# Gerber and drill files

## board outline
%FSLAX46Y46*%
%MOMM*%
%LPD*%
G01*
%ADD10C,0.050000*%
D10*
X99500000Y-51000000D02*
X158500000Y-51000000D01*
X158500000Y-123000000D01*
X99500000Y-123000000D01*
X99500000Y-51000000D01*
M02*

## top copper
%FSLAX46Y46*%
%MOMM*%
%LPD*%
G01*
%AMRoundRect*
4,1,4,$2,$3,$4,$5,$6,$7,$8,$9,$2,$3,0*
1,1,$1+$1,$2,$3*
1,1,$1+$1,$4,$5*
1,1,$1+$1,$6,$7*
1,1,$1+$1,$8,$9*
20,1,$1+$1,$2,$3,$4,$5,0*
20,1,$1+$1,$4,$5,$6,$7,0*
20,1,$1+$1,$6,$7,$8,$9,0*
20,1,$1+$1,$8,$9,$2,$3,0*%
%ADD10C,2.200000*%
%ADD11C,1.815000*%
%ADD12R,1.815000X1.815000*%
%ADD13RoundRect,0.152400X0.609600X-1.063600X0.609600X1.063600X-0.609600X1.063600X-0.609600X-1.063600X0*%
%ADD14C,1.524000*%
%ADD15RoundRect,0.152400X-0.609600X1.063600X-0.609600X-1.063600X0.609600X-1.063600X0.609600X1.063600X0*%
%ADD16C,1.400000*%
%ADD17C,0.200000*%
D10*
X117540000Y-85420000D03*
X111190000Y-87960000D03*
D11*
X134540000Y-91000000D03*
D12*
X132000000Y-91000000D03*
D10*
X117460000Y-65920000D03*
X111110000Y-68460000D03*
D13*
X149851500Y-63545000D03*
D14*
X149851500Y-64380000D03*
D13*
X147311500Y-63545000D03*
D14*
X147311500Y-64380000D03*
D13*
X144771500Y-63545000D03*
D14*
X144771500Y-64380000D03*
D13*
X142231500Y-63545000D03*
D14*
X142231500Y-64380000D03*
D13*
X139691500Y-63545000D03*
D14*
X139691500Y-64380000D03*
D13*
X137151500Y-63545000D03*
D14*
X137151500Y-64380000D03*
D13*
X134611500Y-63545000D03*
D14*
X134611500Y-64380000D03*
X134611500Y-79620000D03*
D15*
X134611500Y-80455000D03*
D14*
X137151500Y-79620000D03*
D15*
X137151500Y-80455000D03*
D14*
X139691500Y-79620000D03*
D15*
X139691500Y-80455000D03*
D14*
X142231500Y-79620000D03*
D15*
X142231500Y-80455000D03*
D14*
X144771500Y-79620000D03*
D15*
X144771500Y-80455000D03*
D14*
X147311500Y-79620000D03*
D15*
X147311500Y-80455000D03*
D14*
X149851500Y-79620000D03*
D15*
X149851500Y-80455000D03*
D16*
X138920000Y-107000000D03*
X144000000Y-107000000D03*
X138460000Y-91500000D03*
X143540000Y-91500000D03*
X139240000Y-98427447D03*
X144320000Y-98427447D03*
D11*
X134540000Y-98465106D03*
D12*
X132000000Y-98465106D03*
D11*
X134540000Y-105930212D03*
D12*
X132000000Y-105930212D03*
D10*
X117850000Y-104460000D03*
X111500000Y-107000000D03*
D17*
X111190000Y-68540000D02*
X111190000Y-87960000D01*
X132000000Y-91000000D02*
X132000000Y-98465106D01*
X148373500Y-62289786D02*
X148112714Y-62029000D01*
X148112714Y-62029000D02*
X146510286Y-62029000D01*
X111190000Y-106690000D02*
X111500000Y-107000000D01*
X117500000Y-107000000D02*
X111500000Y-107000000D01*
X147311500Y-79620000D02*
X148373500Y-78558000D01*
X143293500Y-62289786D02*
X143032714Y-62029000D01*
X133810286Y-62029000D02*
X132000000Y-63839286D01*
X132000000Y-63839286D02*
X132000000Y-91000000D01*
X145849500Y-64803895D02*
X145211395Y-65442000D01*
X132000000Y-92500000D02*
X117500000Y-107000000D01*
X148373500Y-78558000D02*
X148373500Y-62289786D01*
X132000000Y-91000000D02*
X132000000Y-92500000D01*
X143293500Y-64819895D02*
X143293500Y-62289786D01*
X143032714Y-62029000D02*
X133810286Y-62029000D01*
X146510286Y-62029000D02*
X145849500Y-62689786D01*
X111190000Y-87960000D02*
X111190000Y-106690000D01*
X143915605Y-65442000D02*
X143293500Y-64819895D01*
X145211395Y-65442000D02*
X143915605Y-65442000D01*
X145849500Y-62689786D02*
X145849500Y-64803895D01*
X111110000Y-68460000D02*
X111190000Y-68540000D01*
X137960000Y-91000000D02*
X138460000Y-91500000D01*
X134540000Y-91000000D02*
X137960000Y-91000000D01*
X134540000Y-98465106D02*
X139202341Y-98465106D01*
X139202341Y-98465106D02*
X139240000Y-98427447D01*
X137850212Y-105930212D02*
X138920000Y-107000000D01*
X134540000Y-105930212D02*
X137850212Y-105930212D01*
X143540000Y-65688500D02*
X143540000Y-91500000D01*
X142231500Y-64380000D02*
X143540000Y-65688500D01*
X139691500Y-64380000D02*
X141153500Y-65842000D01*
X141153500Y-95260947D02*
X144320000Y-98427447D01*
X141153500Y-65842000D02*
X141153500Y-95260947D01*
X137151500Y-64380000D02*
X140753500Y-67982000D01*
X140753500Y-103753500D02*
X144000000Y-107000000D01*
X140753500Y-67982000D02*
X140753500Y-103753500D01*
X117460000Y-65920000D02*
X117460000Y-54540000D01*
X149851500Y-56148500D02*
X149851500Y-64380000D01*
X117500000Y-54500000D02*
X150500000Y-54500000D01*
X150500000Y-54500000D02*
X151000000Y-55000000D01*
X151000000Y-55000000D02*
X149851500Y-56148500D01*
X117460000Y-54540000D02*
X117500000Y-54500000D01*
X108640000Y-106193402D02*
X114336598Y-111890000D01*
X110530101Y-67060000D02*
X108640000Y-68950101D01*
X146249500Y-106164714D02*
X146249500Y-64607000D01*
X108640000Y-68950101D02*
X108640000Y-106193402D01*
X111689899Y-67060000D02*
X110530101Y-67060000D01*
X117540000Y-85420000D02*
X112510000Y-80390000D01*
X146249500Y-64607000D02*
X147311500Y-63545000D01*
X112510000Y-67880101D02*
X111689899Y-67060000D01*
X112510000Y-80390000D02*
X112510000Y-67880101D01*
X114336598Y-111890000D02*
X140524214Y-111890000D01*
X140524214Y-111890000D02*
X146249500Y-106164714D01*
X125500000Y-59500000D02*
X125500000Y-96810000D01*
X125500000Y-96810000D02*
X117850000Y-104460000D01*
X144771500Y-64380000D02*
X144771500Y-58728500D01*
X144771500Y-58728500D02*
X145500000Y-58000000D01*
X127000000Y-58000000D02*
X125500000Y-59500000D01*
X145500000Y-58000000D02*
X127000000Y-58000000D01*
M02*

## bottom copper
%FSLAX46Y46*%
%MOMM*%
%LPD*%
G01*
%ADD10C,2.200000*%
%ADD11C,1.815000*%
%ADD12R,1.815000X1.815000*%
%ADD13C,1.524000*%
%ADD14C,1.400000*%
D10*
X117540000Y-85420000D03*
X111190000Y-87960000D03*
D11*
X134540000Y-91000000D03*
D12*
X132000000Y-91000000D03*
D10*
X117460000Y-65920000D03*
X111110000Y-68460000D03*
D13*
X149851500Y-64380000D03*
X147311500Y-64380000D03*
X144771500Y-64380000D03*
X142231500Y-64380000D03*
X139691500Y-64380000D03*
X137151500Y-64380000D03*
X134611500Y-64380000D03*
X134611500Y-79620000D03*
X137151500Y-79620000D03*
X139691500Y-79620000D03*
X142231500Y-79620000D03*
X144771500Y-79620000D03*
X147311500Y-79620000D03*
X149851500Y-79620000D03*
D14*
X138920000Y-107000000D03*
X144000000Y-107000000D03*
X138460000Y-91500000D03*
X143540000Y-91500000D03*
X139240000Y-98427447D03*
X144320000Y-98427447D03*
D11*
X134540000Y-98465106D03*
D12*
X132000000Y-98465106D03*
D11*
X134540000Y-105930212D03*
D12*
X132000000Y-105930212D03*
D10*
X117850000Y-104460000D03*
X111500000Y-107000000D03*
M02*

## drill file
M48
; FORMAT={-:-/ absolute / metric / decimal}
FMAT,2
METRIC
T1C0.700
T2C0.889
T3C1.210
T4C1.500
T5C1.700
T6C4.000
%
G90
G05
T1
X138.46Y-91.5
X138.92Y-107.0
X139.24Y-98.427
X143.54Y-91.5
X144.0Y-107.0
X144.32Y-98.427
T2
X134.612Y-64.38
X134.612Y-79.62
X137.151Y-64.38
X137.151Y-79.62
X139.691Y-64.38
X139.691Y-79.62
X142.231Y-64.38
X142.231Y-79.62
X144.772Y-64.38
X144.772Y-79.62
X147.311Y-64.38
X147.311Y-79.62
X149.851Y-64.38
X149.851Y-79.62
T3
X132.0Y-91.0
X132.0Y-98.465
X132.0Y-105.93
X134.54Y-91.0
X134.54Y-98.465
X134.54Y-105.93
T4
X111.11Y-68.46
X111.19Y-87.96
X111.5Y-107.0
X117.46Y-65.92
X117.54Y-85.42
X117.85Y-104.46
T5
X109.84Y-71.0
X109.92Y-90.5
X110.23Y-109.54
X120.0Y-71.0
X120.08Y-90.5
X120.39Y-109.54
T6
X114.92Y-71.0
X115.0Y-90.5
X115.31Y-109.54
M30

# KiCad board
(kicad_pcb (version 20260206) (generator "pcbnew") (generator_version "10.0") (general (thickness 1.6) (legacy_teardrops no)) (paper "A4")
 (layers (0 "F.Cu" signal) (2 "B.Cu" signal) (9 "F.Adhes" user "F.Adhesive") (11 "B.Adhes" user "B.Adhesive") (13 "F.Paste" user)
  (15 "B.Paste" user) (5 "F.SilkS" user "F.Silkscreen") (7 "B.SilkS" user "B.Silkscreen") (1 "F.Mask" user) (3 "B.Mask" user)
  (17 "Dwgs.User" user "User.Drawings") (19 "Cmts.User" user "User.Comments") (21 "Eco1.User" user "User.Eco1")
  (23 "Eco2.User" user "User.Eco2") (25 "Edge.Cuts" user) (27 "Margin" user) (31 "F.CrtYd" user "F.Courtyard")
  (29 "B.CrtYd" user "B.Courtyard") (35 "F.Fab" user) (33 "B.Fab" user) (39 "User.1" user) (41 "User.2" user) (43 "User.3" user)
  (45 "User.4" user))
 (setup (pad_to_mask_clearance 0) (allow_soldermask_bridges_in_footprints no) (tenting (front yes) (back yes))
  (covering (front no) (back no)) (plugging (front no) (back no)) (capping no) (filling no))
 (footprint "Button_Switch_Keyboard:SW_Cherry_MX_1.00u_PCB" (layer "F.Cu") (at 117.54 85.42)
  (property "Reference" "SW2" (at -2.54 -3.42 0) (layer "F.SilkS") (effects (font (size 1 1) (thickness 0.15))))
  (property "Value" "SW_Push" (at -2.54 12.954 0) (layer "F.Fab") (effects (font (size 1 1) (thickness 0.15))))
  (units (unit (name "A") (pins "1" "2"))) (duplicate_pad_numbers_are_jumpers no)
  (pad "" np_thru_hole circle (at -7.62 5.08) (size 1.7 1.7) (drill 1.7) (layers "*.Cu" "*.Mask"))
  (pad "" np_thru_hole circle (at -2.54 5.08) (size 4 4) (drill 4) (layers "*.Cu" "*.Mask"))
  (pad "" np_thru_hole circle (at 2.54 5.08) (size 1.7 1.7) (drill 1.7) (layers "*.Cu" "*.Mask"))
  (pad "1" thru_hole circle (at 0 0) (size 2.2 2.2) (drill 1.5) (layers "*.Cu" "*.Mask") (remove_unused_layers no) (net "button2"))
  (pad "2" thru_hole circle (at -6.35 2.54) (size 2.2 2.2) (drill 1.5) (layers "*.Cu" "*.Mask") (remove_unused_layers no) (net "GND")))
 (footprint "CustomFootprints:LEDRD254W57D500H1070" (layer "F.Cu") (at 133.27 91)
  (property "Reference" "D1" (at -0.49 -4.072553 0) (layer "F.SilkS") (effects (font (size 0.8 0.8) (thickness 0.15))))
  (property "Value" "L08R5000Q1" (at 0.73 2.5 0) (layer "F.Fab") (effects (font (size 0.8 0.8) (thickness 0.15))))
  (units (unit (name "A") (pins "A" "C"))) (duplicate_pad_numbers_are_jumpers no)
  (pad "A" thru_hole circle (at 1.27 0) (size 1.815 1.815) (drill 1.21) (layers "*.Cu" "*.Mask") (remove_unused_layers no)
   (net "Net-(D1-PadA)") (solder_mask_margin 0.102))
  (pad "C" thru_hole rect (at -1.27 0) (size 1.815 1.815) (drill 1.21) (layers "*.Cu" "*.Mask") (remove_unused_layers no) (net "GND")
   (solder_mask_margin 0.102)))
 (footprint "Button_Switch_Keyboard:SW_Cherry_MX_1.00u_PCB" (layer "F.Cu") (at 117.46 65.92)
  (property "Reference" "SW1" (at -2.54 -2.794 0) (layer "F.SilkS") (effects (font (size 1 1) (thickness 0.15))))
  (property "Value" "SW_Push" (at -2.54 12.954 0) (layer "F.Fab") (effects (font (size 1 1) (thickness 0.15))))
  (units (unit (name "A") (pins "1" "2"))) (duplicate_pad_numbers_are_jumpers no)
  (pad "" np_thru_hole circle (at -7.62 5.08) (size 1.7 1.7) (drill 1.7) (layers "*.Cu" "*.Mask"))
  (pad "" np_thru_hole circle (at -2.54 5.08) (size 4 4) (drill 4) (layers "*.Cu" "*.Mask"))
  (pad "" np_thru_hole circle (at 2.54 5.08) (size 1.7 1.7) (drill 1.7) (layers "*.Cu" "*.Mask"))
  (pad "1" thru_hole circle (at 0 0) (size 2.2 2.2) (drill 1.5) (layers "*.Cu" "*.Mask") (remove_unused_layers no) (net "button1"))
  (pad "2" thru_hole circle (at -6.35 2.54) (size 2.2 2.2) (drill 1.5) (layers "*.Cu" "*.Mask") (remove_unused_layers no) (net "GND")))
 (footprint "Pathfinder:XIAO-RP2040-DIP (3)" (layer "F.Cu") (at 142.2315 72)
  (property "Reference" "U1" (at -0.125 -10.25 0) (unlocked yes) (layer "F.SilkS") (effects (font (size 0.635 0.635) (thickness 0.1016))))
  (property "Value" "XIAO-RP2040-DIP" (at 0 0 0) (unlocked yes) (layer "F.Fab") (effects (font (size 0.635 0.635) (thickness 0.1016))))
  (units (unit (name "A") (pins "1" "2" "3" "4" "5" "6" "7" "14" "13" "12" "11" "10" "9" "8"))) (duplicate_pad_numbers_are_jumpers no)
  (pad "1" smd roundrect (at 7.62 -8.455 90) (size 2.432 1.524) (layers "F.Cu" "F.Mask") (roundrect_rratio 0.1) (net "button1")
   (thermal_bridge_angle 45))
  (pad "1" thru_hole circle (at 7.62 -7.62 90) (size 1.524 1.524) (drill 0.889) (layers "*.Cu" "*.Mask") (remove_unused_layers no)
   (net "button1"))
  (pad "2" smd roundrect (at 5.08 -8.455 90) (size 2.432 1.524) (layers "F.Cu" "F.Mask") (roundrect_rratio 0.1) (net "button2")
   (thermal_bridge_angle 45))
  (pad "2" thru_hole circle (at 5.08 -7.62 90) (size 1.524 1.524) (drill 0.889) (layers "*.Cu" "*.Mask") (remove_unused_layers no)
   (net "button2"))
  (pad "3" smd roundrect (at 2.54 -8.455 90) (size 2.432 1.524) (layers "F.Cu" "F.Mask") (roundrect_rratio 0.1) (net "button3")
   (thermal_bridge_angle 45))
  (pad "3" thru_hole circle (at 2.54 -7.62 90) (size 1.524 1.524) (drill 0.889) (layers "*.Cu" "*.Mask") (remove_unused_layers no)
   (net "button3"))
  (pad "4" smd roundrect (at 0 -8.455 90) (size 2.432 1.524) (layers "F.Cu" "F.Mask") (roundrect_rratio 0.1) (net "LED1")
   (thermal_bridge_angle 45))
  (pad "4" thru_hole circle (at 0 -7.62 90) (size 1.524 1.524) (drill 0.889) (layers "*.Cu" "*.Mask") (remove_unused_layers no) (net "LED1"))
  (pad "5" smd roundrect (at -2.54 -8.455 90) (size 2.432 1.524) (layers "F.Cu" "F.Mask") (roundrect_rratio 0.1) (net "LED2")
   (thermal_bridge_angle 45))
  (pad "5" thru_hole circle (at -2.54 -7.62 90) (size 1.524 1.524) (drill 0.889) (layers "*.Cu" "*.Mask") (remove_unused_layers no)
   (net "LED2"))
  (pad "6" smd roundrect (at -5.08 -8.455 90) (size 2.432 1.524) (layers "F.Cu" "F.Mask") (roundrect_rratio 0.1) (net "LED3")
   (thermal_bridge_angle 45))
  (pad "6" thru_hole circle (at -5.08 -7.62 90) (size 1.524 1.524) (drill 0.889) (layers "*.Cu" "*.Mask") (remove_unused_layers no)
   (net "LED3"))
  (pad "7" smd roundrect (at -7.62 -8.455 90) (size 2.432 1.524) (layers "F.Cu" "F.Mask") (roundrect_rratio 0.1)
   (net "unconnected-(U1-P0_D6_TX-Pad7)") (thermal_bridge_angle 45))
  (pad "7" thru_hole circle (at -7.62 -7.62 90) (size 1.524 1.524) (drill 0.889) (layers "*.Cu" "*.Mask") (remove_unused_layers no)
   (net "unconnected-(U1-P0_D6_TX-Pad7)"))
  (pad "8" thru_hole circle (at -7.62 7.62 270) (size 1.524 1.524) (drill 0.889) (layers "*.Cu" "*.Mask") (remove_unused_layers no)
   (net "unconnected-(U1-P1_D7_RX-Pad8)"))
  (pad "8" smd roundrect (at -7.62 8.455 270) (size 2.432 1.524) (layers "F.Cu" "F.Mask") (roundrect_rratio 0.1)
   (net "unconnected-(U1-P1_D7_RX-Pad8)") (thermal_bridge_angle 45))
  (pad "9" thru_hole circle (at -5.08 7.62 270) (size 1.524 1.524) (drill 0.889) (layers "*.Cu" "*.Mask") (remove_unused_layers no)
   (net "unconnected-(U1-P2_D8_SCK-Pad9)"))
  (pad "9" smd roundrect (at -5.08 8.455 270) (size 2.432 1.524) (layers "F.Cu" "F.Mask") (roundrect_rratio 0.1)
   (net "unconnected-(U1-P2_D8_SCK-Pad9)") (thermal_bridge_angle 45))
  (pad "10" thru_hole circle (at -2.54 7.62 270) (size 1.524 1.524) (drill 0.889) (layers "*.Cu" "*.Mask") (remove_unused_layers no)
   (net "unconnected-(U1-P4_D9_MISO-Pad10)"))
  (pad "10" smd roundrect (at -2.54 8.455 270) (size 2.432 1.524) (layers "F.Cu" "F.Mask") (roundrect_rratio 0.1)
   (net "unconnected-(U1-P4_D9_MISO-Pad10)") (thermal_bridge_angle 45))
  (pad "11" thru_hole circle (at 0 7.62 270) (size 1.524 1.524) (drill 0.889) (layers "*.Cu" "*.Mask") (remove_unused_layers no)
   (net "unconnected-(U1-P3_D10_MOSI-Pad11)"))
  (pad "11" smd roundrect (at 0 8.455 270) (size 2.432 1.524) (layers "F.Cu" "F.Mask") (roundrect_rratio 0.1)
   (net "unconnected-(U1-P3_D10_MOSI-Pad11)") (thermal_bridge_angle 45))
  (pad "12" thru_hole circle (at 2.54 7.62 270) (size 1.524 1.524) (drill 0.889) (layers "*.Cu" "*.Mask") (remove_unused_layers no)
   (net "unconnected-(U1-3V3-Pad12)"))
  (pad "12" smd roundrect (at 2.54 8.455 270) (size 2.432 1.524) (layers "F.Cu" "F.Mask") (roundrect_rratio 0.1)
   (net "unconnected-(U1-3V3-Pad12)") (thermal_bridge_angle 45))
  (pad "13" thru_hole circle (at 5.08 7.62 270) (size 1.524 1.524) (drill 0.889) (layers "*.Cu" "*.Mask") (remove_unused_layers no)
   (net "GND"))
  (pad "13" smd roundrect (at 5.08 8.455 270) (size 2.432 1.524) (layers "F.Cu" "F.Mask") (roundrect_rratio 0.1) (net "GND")
   (thermal_bridge_angle 45))
  (pad "14" thru_hole circle (at 7.62 7.62 270) (size 1.524 1.524) (drill 0.889) (layers "*.Cu" "*.Mask") (remove_unused_layers no)
   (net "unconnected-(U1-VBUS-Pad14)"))
  (pad "14" smd roundrect (at 7.62 8.455 270) (size 2.432 1.524) (layers "F.Cu" "F.Mask") (roundrect_rratio 0.1)
   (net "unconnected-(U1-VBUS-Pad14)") (thermal_bridge_angle 45)))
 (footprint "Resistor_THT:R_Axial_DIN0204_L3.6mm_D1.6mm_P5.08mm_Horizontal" (layer "F.Cu") (at 138.92 107)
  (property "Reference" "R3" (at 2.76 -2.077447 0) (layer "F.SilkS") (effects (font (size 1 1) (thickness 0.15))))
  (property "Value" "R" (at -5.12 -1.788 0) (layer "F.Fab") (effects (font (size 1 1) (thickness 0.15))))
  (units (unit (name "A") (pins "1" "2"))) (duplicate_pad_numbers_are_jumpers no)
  (pad "1" thru_hole circle (at 0 0) (size 1.4 1.4) (drill 0.7) (layers "*.Cu" "*.Mask") (remove_unused_layers no) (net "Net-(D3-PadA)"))
  (pad "2" thru_hole circle (at 5.08 0) (size 1.4 1.4) (drill 0.7) (layers "*.Cu" "*.Mask") (remove_unused_layers no) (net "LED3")))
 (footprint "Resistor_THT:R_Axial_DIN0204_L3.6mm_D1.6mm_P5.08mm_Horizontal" (layer "F.Cu") (at 138.46 91.5)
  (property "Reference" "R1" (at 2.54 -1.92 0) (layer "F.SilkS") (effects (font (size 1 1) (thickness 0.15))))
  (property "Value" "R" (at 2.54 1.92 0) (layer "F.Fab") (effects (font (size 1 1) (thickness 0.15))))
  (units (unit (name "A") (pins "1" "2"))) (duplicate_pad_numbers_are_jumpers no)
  (pad "1" thru_hole circle (at 0 0) (size 1.4 1.4) (drill 0.7) (layers "*.Cu" "*.Mask") (remove_unused_layers no) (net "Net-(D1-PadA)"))
  (pad "2" thru_hole circle (at 5.08 0) (size 1.4 1.4) (drill 0.7) (layers "*.Cu" "*.Mask") (remove_unused_layers no) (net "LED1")))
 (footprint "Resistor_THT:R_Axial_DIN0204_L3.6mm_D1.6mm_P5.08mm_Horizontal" (layer "F.Cu") (at 139.24 98.427447)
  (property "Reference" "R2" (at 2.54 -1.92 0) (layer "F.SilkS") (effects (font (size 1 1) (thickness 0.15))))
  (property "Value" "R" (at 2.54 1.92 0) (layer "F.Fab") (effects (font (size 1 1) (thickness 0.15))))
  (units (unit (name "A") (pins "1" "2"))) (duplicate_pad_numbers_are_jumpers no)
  (pad "1" thru_hole circle (at 0 0) (size 1.4 1.4) (drill 0.7) (layers "*.Cu" "*.Mask") (remove_unused_layers no) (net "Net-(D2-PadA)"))
  (pad "2" thru_hole circle (at 5.08 0) (size 1.4 1.4) (drill 0.7) (layers "*.Cu" "*.Mask") (remove_unused_layers no) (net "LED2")))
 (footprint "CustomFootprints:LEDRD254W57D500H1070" (layer "F.Cu") (at 133.27 98.465106)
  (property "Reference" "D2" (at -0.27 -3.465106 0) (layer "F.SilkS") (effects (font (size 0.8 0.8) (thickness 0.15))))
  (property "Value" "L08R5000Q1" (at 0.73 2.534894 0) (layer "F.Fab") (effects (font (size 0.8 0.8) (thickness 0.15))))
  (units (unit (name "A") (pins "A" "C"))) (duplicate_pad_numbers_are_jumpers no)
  (pad "A" thru_hole circle (at 1.27 0) (size 1.815 1.815) (drill 1.21) (layers "*.Cu" "*.Mask") (remove_unused_layers no)
   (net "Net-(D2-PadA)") (solder_mask_margin 0.102))
  (pad "C" thru_hole rect (at -1.27 0) (size 1.815 1.815) (drill 1.21) (layers "*.Cu" "*.Mask") (remove_unused_layers no) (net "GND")
   (solder_mask_margin 0.102)))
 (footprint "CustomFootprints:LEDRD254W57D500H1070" (layer "F.Cu") (at 133.27 105.930212)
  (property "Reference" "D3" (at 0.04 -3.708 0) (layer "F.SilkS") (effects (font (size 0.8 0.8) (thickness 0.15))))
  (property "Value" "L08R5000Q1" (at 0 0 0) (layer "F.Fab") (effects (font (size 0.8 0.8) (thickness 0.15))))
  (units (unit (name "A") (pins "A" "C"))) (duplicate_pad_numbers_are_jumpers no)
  (pad "A" thru_hole circle (at 1.27 0) (size 1.815 1.815) (drill 1.21) (layers "*.Cu" "*.Mask") (remove_unused_layers no)
   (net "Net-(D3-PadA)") (solder_mask_margin 0.102))
  (pad "C" thru_hole rect (at -1.27 0) (size 1.815 1.815) (drill 1.21) (layers "*.Cu" "*.Mask") (remove_unused_layers no)
   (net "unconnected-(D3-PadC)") (solder_mask_margin 0.102)))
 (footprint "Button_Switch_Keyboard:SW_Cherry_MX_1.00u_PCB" (layer "F.Cu") (at 117.85 104.46)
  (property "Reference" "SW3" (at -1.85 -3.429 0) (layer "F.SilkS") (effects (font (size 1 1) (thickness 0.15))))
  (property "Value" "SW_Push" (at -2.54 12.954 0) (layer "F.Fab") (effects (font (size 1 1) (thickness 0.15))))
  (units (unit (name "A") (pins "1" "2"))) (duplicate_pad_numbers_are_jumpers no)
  (pad "" np_thru_hole circle (at -7.62 5.08) (size 1.7 1.7) (drill 1.7) (layers "*.Cu" "*.Mask"))
  (pad "" np_thru_hole circle (at -2.54 5.08) (size 4 4) (drill 4) (layers "*.Cu" "*.Mask"))
  (pad "" np_thru_hole circle (at 2.54 5.08) (size 1.7 1.7) (drill 1.7) (layers "*.Cu" "*.Mask"))
  (pad "1" thru_hole circle (at 0 0) (size 2.2 2.2) (drill 1.5) (layers "*.Cu" "*.Mask") (remove_unused_layers no) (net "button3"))
  (pad "2" thru_hole circle (at -6.35 2.54) (size 2.2 2.2) (drill 1.5) (layers "*.Cu" "*.Mask") (remove_unused_layers no) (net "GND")))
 (gr_rect (start 99.5 51) (end 158.5 123) (stroke (width 0.05) (type default)) (fill no) (layer "Edge.Cuts"))
 (segment (start 111.19 68.54) (end 111.19 87.96) (width 0.2) (layer "F.Cu") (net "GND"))
 (segment (start 132 91) (end 132 98.465106) (width 0.2) (layer "F.Cu") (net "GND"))
 (segment (start 148.3735 62.289786) (end 148.112714 62.029) (width 0.2) (layer "F.Cu") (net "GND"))
 (segment (start 148.112714 62.029) (end 146.510286 62.029) (width 0.2) (layer "F.Cu") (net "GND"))
 (segment (start 111.19 106.69) (end 111.5 107) (width 0.2) (layer "F.Cu") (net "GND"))
 (segment (start 117.5 107) (end 111.5 107) (width 0.2) (layer "F.Cu") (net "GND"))
 (segment (start 147.3115 79.62) (end 148.3735 78.558) (width 0.2) (layer "F.Cu") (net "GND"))
 (segment (start 143.2935 62.289786) (end 143.032714 62.029) (width 0.2) (layer "F.Cu") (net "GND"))
 (segment (start 133.810286 62.029) (end 132 63.839286) (width 0.2) (layer "F.Cu") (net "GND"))
 (segment (start 132 63.839286) (end 132 91) (width 0.2) (layer "F.Cu") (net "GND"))
 (segment (start 145.8495 64.803895) (end 145.211395 65.442) (width 0.2) (layer "F.Cu") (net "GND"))
 (segment (start 132 92.5) (end 117.5 107) (width 0.2) (layer "F.Cu") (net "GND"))
 (segment (start 148.3735 78.558) (end 148.3735 62.289786) (width 0.2) (layer "F.Cu") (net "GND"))
 (segment (start 132 91) (end 132 92.5) (width 0.2) (layer "F.Cu") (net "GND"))
 (segment (start 143.2935 64.819895) (end 143.2935 62.289786) (width 0.2) (layer "F.Cu") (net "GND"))
 (segment (start 143.032714 62.029) (end 133.810286 62.029) (width 0.2) (layer "F.Cu") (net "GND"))
 (segment (start 146.510286 62.029) (end 145.8495 62.689786) (width 0.2) (layer "F.Cu") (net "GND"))
 (segment (start 111.19 87.96) (end 111.19 106.69) (width 0.2) (layer "F.Cu") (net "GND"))
 (segment (start 143.915605 65.442) (end 143.2935 64.819895) (width 0.2) (layer "F.Cu") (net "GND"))
 (segment (start 145.211395 65.442) (end 143.915605 65.442) (width 0.2) (layer "F.Cu") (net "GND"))
 (segment (start 145.8495 62.689786) (end 145.8495 64.803895) (width 0.2) (layer "F.Cu") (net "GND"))
 (segment (start 111.11 68.46) (end 111.19 68.54) (width 0.2) (layer "F.Cu") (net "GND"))
 (segment (start 137.96 91) (end 138.46 91.5) (width 0.2) (layer "F.Cu") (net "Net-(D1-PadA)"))
 (segment (start 134.54 91) (end 137.96 91) (width 0.2) (layer "F.Cu") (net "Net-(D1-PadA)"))
 (segment (start 134.54 98.465106) (end 139.202341 98.465106) (width 0.2) (layer "F.Cu") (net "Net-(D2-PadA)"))
 (segment (start 139.202341 98.465106) (end 139.24 98.427447) (width 0.2) (layer "F.Cu") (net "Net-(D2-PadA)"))
 (segment (start 137.850212 105.930212) (end 138.92 107) (width 0.2) (layer "F.Cu") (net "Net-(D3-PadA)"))
 (segment (start 134.54 105.930212) (end 137.850212 105.930212) (width 0.2) (layer "F.Cu") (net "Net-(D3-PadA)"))
 (segment (start 143.54 65.6885) (end 143.54 91.5) (width 0.2) (layer "F.Cu") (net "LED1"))
 (segment (start 142.2315 64.38) (end 143.54 65.6885) (width 0.2) (layer "F.Cu") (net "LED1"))
 (segment (start 139.6915 64.38) (end 141.1535 65.842) (width 0.2) (layer "F.Cu") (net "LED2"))
 (segment (start 141.1535 95.260947) (end 144.32 98.427447) (width 0.2) (layer "F.Cu") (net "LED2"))
 (segment (start 141.1535 65.842) (end 141.1535 95.260947) (width 0.2) (layer "F.Cu") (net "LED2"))
 (segment (start 137.1515 64.38) (end 140.7535 67.982) (width 0.2) (layer "F.Cu") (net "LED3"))
 (segment (start 140.7535 103.7535) (end 144 107) (width 0.2) (layer "F.Cu") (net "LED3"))
 (segment (start 140.7535 67.982) (end 140.7535 103.7535) (width 0.2) (layer "F.Cu") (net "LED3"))
 (segment (start 117.46 65.92) (end 117.46 54.54) (width 0.2) (layer "F.Cu") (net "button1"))
 (segment (start 149.8515 56.1485) (end 149.8515 64.38) (width 0.2) (layer "F.Cu") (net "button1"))
 (segment (start 117.5 54.5) (end 150.5 54.5) (width 0.2) (layer "F.Cu") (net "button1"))
 (segment (start 150.5 54.5) (end 151 55) (width 0.2) (layer "F.Cu") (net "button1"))
 (segment (start 151 55) (end 149.8515 56.1485) (width 0.2) (layer "F.Cu") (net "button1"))
 (segment (start 117.46 54.54) (end 117.5 54.5) (width 0.2) (layer "F.Cu") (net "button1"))
 (segment (start 108.64 106.193402) (end 114.336598 111.89) (width 0.2) (layer "F.Cu") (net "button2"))
 (segment (start 110.530101 67.06) (end 108.64 68.950101) (width 0.2) (layer "F.Cu") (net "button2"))
 (segment (start 146.2495 106.164714) (end 146.2495 64.607) (width 0.2) (layer "F.Cu") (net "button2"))
 (segment (start 108.64 68.950101) (end 108.64 106.193402) (width 0.2) (layer "F.Cu") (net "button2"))
 (segment (start 111.689899 67.06) (end 110.530101 67.06) (width 0.2) (layer "F.Cu") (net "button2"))
 (segment (start 117.54 85.42) (end 112.51 80.39) (width 0.2) (layer "F.Cu") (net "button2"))
 (segment (start 146.2495 64.607) (end 147.3115 63.545) (width 0.2) (layer "F.Cu") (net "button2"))
 (segment (start 112.51 67.880101) (end 111.689899 67.06) (width 0.2) (layer "F.Cu") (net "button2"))
 (segment (start 112.51 80.39) (end 112.51 67.880101) (width 0.2) (layer "F.Cu") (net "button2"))
 (segment (start 114.336598 111.89) (end 140.524214 111.89) (width 0.2) (layer "F.Cu") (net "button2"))
 (segment (start 140.524214 111.89) (end 146.2495 106.164714) (width 0.2) (layer "F.Cu") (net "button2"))
 (segment (start 125.5 59.5) (end 125.5 96.81) (width 0.2) (layer "F.Cu") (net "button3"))
 (segment (start 125.5 96.81) (end 117.85 104.46) (width 0.2) (layer "F.Cu") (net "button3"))
 (segment (start 144.7715 64.38) (end 144.7715 58.7285) (width 0.2) (layer "F.Cu") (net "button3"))
 (segment (start 144.7715 58.7285) (end 145.5 58) (width 0.2) (layer "F.Cu") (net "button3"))
 (segment (start 127 58) (end 125.5 59.5) (width 0.2) (layer "F.Cu") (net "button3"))
 (segment (start 145.5 58) (end 127 58) (width 0.2) (layer "F.Cu") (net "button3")))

